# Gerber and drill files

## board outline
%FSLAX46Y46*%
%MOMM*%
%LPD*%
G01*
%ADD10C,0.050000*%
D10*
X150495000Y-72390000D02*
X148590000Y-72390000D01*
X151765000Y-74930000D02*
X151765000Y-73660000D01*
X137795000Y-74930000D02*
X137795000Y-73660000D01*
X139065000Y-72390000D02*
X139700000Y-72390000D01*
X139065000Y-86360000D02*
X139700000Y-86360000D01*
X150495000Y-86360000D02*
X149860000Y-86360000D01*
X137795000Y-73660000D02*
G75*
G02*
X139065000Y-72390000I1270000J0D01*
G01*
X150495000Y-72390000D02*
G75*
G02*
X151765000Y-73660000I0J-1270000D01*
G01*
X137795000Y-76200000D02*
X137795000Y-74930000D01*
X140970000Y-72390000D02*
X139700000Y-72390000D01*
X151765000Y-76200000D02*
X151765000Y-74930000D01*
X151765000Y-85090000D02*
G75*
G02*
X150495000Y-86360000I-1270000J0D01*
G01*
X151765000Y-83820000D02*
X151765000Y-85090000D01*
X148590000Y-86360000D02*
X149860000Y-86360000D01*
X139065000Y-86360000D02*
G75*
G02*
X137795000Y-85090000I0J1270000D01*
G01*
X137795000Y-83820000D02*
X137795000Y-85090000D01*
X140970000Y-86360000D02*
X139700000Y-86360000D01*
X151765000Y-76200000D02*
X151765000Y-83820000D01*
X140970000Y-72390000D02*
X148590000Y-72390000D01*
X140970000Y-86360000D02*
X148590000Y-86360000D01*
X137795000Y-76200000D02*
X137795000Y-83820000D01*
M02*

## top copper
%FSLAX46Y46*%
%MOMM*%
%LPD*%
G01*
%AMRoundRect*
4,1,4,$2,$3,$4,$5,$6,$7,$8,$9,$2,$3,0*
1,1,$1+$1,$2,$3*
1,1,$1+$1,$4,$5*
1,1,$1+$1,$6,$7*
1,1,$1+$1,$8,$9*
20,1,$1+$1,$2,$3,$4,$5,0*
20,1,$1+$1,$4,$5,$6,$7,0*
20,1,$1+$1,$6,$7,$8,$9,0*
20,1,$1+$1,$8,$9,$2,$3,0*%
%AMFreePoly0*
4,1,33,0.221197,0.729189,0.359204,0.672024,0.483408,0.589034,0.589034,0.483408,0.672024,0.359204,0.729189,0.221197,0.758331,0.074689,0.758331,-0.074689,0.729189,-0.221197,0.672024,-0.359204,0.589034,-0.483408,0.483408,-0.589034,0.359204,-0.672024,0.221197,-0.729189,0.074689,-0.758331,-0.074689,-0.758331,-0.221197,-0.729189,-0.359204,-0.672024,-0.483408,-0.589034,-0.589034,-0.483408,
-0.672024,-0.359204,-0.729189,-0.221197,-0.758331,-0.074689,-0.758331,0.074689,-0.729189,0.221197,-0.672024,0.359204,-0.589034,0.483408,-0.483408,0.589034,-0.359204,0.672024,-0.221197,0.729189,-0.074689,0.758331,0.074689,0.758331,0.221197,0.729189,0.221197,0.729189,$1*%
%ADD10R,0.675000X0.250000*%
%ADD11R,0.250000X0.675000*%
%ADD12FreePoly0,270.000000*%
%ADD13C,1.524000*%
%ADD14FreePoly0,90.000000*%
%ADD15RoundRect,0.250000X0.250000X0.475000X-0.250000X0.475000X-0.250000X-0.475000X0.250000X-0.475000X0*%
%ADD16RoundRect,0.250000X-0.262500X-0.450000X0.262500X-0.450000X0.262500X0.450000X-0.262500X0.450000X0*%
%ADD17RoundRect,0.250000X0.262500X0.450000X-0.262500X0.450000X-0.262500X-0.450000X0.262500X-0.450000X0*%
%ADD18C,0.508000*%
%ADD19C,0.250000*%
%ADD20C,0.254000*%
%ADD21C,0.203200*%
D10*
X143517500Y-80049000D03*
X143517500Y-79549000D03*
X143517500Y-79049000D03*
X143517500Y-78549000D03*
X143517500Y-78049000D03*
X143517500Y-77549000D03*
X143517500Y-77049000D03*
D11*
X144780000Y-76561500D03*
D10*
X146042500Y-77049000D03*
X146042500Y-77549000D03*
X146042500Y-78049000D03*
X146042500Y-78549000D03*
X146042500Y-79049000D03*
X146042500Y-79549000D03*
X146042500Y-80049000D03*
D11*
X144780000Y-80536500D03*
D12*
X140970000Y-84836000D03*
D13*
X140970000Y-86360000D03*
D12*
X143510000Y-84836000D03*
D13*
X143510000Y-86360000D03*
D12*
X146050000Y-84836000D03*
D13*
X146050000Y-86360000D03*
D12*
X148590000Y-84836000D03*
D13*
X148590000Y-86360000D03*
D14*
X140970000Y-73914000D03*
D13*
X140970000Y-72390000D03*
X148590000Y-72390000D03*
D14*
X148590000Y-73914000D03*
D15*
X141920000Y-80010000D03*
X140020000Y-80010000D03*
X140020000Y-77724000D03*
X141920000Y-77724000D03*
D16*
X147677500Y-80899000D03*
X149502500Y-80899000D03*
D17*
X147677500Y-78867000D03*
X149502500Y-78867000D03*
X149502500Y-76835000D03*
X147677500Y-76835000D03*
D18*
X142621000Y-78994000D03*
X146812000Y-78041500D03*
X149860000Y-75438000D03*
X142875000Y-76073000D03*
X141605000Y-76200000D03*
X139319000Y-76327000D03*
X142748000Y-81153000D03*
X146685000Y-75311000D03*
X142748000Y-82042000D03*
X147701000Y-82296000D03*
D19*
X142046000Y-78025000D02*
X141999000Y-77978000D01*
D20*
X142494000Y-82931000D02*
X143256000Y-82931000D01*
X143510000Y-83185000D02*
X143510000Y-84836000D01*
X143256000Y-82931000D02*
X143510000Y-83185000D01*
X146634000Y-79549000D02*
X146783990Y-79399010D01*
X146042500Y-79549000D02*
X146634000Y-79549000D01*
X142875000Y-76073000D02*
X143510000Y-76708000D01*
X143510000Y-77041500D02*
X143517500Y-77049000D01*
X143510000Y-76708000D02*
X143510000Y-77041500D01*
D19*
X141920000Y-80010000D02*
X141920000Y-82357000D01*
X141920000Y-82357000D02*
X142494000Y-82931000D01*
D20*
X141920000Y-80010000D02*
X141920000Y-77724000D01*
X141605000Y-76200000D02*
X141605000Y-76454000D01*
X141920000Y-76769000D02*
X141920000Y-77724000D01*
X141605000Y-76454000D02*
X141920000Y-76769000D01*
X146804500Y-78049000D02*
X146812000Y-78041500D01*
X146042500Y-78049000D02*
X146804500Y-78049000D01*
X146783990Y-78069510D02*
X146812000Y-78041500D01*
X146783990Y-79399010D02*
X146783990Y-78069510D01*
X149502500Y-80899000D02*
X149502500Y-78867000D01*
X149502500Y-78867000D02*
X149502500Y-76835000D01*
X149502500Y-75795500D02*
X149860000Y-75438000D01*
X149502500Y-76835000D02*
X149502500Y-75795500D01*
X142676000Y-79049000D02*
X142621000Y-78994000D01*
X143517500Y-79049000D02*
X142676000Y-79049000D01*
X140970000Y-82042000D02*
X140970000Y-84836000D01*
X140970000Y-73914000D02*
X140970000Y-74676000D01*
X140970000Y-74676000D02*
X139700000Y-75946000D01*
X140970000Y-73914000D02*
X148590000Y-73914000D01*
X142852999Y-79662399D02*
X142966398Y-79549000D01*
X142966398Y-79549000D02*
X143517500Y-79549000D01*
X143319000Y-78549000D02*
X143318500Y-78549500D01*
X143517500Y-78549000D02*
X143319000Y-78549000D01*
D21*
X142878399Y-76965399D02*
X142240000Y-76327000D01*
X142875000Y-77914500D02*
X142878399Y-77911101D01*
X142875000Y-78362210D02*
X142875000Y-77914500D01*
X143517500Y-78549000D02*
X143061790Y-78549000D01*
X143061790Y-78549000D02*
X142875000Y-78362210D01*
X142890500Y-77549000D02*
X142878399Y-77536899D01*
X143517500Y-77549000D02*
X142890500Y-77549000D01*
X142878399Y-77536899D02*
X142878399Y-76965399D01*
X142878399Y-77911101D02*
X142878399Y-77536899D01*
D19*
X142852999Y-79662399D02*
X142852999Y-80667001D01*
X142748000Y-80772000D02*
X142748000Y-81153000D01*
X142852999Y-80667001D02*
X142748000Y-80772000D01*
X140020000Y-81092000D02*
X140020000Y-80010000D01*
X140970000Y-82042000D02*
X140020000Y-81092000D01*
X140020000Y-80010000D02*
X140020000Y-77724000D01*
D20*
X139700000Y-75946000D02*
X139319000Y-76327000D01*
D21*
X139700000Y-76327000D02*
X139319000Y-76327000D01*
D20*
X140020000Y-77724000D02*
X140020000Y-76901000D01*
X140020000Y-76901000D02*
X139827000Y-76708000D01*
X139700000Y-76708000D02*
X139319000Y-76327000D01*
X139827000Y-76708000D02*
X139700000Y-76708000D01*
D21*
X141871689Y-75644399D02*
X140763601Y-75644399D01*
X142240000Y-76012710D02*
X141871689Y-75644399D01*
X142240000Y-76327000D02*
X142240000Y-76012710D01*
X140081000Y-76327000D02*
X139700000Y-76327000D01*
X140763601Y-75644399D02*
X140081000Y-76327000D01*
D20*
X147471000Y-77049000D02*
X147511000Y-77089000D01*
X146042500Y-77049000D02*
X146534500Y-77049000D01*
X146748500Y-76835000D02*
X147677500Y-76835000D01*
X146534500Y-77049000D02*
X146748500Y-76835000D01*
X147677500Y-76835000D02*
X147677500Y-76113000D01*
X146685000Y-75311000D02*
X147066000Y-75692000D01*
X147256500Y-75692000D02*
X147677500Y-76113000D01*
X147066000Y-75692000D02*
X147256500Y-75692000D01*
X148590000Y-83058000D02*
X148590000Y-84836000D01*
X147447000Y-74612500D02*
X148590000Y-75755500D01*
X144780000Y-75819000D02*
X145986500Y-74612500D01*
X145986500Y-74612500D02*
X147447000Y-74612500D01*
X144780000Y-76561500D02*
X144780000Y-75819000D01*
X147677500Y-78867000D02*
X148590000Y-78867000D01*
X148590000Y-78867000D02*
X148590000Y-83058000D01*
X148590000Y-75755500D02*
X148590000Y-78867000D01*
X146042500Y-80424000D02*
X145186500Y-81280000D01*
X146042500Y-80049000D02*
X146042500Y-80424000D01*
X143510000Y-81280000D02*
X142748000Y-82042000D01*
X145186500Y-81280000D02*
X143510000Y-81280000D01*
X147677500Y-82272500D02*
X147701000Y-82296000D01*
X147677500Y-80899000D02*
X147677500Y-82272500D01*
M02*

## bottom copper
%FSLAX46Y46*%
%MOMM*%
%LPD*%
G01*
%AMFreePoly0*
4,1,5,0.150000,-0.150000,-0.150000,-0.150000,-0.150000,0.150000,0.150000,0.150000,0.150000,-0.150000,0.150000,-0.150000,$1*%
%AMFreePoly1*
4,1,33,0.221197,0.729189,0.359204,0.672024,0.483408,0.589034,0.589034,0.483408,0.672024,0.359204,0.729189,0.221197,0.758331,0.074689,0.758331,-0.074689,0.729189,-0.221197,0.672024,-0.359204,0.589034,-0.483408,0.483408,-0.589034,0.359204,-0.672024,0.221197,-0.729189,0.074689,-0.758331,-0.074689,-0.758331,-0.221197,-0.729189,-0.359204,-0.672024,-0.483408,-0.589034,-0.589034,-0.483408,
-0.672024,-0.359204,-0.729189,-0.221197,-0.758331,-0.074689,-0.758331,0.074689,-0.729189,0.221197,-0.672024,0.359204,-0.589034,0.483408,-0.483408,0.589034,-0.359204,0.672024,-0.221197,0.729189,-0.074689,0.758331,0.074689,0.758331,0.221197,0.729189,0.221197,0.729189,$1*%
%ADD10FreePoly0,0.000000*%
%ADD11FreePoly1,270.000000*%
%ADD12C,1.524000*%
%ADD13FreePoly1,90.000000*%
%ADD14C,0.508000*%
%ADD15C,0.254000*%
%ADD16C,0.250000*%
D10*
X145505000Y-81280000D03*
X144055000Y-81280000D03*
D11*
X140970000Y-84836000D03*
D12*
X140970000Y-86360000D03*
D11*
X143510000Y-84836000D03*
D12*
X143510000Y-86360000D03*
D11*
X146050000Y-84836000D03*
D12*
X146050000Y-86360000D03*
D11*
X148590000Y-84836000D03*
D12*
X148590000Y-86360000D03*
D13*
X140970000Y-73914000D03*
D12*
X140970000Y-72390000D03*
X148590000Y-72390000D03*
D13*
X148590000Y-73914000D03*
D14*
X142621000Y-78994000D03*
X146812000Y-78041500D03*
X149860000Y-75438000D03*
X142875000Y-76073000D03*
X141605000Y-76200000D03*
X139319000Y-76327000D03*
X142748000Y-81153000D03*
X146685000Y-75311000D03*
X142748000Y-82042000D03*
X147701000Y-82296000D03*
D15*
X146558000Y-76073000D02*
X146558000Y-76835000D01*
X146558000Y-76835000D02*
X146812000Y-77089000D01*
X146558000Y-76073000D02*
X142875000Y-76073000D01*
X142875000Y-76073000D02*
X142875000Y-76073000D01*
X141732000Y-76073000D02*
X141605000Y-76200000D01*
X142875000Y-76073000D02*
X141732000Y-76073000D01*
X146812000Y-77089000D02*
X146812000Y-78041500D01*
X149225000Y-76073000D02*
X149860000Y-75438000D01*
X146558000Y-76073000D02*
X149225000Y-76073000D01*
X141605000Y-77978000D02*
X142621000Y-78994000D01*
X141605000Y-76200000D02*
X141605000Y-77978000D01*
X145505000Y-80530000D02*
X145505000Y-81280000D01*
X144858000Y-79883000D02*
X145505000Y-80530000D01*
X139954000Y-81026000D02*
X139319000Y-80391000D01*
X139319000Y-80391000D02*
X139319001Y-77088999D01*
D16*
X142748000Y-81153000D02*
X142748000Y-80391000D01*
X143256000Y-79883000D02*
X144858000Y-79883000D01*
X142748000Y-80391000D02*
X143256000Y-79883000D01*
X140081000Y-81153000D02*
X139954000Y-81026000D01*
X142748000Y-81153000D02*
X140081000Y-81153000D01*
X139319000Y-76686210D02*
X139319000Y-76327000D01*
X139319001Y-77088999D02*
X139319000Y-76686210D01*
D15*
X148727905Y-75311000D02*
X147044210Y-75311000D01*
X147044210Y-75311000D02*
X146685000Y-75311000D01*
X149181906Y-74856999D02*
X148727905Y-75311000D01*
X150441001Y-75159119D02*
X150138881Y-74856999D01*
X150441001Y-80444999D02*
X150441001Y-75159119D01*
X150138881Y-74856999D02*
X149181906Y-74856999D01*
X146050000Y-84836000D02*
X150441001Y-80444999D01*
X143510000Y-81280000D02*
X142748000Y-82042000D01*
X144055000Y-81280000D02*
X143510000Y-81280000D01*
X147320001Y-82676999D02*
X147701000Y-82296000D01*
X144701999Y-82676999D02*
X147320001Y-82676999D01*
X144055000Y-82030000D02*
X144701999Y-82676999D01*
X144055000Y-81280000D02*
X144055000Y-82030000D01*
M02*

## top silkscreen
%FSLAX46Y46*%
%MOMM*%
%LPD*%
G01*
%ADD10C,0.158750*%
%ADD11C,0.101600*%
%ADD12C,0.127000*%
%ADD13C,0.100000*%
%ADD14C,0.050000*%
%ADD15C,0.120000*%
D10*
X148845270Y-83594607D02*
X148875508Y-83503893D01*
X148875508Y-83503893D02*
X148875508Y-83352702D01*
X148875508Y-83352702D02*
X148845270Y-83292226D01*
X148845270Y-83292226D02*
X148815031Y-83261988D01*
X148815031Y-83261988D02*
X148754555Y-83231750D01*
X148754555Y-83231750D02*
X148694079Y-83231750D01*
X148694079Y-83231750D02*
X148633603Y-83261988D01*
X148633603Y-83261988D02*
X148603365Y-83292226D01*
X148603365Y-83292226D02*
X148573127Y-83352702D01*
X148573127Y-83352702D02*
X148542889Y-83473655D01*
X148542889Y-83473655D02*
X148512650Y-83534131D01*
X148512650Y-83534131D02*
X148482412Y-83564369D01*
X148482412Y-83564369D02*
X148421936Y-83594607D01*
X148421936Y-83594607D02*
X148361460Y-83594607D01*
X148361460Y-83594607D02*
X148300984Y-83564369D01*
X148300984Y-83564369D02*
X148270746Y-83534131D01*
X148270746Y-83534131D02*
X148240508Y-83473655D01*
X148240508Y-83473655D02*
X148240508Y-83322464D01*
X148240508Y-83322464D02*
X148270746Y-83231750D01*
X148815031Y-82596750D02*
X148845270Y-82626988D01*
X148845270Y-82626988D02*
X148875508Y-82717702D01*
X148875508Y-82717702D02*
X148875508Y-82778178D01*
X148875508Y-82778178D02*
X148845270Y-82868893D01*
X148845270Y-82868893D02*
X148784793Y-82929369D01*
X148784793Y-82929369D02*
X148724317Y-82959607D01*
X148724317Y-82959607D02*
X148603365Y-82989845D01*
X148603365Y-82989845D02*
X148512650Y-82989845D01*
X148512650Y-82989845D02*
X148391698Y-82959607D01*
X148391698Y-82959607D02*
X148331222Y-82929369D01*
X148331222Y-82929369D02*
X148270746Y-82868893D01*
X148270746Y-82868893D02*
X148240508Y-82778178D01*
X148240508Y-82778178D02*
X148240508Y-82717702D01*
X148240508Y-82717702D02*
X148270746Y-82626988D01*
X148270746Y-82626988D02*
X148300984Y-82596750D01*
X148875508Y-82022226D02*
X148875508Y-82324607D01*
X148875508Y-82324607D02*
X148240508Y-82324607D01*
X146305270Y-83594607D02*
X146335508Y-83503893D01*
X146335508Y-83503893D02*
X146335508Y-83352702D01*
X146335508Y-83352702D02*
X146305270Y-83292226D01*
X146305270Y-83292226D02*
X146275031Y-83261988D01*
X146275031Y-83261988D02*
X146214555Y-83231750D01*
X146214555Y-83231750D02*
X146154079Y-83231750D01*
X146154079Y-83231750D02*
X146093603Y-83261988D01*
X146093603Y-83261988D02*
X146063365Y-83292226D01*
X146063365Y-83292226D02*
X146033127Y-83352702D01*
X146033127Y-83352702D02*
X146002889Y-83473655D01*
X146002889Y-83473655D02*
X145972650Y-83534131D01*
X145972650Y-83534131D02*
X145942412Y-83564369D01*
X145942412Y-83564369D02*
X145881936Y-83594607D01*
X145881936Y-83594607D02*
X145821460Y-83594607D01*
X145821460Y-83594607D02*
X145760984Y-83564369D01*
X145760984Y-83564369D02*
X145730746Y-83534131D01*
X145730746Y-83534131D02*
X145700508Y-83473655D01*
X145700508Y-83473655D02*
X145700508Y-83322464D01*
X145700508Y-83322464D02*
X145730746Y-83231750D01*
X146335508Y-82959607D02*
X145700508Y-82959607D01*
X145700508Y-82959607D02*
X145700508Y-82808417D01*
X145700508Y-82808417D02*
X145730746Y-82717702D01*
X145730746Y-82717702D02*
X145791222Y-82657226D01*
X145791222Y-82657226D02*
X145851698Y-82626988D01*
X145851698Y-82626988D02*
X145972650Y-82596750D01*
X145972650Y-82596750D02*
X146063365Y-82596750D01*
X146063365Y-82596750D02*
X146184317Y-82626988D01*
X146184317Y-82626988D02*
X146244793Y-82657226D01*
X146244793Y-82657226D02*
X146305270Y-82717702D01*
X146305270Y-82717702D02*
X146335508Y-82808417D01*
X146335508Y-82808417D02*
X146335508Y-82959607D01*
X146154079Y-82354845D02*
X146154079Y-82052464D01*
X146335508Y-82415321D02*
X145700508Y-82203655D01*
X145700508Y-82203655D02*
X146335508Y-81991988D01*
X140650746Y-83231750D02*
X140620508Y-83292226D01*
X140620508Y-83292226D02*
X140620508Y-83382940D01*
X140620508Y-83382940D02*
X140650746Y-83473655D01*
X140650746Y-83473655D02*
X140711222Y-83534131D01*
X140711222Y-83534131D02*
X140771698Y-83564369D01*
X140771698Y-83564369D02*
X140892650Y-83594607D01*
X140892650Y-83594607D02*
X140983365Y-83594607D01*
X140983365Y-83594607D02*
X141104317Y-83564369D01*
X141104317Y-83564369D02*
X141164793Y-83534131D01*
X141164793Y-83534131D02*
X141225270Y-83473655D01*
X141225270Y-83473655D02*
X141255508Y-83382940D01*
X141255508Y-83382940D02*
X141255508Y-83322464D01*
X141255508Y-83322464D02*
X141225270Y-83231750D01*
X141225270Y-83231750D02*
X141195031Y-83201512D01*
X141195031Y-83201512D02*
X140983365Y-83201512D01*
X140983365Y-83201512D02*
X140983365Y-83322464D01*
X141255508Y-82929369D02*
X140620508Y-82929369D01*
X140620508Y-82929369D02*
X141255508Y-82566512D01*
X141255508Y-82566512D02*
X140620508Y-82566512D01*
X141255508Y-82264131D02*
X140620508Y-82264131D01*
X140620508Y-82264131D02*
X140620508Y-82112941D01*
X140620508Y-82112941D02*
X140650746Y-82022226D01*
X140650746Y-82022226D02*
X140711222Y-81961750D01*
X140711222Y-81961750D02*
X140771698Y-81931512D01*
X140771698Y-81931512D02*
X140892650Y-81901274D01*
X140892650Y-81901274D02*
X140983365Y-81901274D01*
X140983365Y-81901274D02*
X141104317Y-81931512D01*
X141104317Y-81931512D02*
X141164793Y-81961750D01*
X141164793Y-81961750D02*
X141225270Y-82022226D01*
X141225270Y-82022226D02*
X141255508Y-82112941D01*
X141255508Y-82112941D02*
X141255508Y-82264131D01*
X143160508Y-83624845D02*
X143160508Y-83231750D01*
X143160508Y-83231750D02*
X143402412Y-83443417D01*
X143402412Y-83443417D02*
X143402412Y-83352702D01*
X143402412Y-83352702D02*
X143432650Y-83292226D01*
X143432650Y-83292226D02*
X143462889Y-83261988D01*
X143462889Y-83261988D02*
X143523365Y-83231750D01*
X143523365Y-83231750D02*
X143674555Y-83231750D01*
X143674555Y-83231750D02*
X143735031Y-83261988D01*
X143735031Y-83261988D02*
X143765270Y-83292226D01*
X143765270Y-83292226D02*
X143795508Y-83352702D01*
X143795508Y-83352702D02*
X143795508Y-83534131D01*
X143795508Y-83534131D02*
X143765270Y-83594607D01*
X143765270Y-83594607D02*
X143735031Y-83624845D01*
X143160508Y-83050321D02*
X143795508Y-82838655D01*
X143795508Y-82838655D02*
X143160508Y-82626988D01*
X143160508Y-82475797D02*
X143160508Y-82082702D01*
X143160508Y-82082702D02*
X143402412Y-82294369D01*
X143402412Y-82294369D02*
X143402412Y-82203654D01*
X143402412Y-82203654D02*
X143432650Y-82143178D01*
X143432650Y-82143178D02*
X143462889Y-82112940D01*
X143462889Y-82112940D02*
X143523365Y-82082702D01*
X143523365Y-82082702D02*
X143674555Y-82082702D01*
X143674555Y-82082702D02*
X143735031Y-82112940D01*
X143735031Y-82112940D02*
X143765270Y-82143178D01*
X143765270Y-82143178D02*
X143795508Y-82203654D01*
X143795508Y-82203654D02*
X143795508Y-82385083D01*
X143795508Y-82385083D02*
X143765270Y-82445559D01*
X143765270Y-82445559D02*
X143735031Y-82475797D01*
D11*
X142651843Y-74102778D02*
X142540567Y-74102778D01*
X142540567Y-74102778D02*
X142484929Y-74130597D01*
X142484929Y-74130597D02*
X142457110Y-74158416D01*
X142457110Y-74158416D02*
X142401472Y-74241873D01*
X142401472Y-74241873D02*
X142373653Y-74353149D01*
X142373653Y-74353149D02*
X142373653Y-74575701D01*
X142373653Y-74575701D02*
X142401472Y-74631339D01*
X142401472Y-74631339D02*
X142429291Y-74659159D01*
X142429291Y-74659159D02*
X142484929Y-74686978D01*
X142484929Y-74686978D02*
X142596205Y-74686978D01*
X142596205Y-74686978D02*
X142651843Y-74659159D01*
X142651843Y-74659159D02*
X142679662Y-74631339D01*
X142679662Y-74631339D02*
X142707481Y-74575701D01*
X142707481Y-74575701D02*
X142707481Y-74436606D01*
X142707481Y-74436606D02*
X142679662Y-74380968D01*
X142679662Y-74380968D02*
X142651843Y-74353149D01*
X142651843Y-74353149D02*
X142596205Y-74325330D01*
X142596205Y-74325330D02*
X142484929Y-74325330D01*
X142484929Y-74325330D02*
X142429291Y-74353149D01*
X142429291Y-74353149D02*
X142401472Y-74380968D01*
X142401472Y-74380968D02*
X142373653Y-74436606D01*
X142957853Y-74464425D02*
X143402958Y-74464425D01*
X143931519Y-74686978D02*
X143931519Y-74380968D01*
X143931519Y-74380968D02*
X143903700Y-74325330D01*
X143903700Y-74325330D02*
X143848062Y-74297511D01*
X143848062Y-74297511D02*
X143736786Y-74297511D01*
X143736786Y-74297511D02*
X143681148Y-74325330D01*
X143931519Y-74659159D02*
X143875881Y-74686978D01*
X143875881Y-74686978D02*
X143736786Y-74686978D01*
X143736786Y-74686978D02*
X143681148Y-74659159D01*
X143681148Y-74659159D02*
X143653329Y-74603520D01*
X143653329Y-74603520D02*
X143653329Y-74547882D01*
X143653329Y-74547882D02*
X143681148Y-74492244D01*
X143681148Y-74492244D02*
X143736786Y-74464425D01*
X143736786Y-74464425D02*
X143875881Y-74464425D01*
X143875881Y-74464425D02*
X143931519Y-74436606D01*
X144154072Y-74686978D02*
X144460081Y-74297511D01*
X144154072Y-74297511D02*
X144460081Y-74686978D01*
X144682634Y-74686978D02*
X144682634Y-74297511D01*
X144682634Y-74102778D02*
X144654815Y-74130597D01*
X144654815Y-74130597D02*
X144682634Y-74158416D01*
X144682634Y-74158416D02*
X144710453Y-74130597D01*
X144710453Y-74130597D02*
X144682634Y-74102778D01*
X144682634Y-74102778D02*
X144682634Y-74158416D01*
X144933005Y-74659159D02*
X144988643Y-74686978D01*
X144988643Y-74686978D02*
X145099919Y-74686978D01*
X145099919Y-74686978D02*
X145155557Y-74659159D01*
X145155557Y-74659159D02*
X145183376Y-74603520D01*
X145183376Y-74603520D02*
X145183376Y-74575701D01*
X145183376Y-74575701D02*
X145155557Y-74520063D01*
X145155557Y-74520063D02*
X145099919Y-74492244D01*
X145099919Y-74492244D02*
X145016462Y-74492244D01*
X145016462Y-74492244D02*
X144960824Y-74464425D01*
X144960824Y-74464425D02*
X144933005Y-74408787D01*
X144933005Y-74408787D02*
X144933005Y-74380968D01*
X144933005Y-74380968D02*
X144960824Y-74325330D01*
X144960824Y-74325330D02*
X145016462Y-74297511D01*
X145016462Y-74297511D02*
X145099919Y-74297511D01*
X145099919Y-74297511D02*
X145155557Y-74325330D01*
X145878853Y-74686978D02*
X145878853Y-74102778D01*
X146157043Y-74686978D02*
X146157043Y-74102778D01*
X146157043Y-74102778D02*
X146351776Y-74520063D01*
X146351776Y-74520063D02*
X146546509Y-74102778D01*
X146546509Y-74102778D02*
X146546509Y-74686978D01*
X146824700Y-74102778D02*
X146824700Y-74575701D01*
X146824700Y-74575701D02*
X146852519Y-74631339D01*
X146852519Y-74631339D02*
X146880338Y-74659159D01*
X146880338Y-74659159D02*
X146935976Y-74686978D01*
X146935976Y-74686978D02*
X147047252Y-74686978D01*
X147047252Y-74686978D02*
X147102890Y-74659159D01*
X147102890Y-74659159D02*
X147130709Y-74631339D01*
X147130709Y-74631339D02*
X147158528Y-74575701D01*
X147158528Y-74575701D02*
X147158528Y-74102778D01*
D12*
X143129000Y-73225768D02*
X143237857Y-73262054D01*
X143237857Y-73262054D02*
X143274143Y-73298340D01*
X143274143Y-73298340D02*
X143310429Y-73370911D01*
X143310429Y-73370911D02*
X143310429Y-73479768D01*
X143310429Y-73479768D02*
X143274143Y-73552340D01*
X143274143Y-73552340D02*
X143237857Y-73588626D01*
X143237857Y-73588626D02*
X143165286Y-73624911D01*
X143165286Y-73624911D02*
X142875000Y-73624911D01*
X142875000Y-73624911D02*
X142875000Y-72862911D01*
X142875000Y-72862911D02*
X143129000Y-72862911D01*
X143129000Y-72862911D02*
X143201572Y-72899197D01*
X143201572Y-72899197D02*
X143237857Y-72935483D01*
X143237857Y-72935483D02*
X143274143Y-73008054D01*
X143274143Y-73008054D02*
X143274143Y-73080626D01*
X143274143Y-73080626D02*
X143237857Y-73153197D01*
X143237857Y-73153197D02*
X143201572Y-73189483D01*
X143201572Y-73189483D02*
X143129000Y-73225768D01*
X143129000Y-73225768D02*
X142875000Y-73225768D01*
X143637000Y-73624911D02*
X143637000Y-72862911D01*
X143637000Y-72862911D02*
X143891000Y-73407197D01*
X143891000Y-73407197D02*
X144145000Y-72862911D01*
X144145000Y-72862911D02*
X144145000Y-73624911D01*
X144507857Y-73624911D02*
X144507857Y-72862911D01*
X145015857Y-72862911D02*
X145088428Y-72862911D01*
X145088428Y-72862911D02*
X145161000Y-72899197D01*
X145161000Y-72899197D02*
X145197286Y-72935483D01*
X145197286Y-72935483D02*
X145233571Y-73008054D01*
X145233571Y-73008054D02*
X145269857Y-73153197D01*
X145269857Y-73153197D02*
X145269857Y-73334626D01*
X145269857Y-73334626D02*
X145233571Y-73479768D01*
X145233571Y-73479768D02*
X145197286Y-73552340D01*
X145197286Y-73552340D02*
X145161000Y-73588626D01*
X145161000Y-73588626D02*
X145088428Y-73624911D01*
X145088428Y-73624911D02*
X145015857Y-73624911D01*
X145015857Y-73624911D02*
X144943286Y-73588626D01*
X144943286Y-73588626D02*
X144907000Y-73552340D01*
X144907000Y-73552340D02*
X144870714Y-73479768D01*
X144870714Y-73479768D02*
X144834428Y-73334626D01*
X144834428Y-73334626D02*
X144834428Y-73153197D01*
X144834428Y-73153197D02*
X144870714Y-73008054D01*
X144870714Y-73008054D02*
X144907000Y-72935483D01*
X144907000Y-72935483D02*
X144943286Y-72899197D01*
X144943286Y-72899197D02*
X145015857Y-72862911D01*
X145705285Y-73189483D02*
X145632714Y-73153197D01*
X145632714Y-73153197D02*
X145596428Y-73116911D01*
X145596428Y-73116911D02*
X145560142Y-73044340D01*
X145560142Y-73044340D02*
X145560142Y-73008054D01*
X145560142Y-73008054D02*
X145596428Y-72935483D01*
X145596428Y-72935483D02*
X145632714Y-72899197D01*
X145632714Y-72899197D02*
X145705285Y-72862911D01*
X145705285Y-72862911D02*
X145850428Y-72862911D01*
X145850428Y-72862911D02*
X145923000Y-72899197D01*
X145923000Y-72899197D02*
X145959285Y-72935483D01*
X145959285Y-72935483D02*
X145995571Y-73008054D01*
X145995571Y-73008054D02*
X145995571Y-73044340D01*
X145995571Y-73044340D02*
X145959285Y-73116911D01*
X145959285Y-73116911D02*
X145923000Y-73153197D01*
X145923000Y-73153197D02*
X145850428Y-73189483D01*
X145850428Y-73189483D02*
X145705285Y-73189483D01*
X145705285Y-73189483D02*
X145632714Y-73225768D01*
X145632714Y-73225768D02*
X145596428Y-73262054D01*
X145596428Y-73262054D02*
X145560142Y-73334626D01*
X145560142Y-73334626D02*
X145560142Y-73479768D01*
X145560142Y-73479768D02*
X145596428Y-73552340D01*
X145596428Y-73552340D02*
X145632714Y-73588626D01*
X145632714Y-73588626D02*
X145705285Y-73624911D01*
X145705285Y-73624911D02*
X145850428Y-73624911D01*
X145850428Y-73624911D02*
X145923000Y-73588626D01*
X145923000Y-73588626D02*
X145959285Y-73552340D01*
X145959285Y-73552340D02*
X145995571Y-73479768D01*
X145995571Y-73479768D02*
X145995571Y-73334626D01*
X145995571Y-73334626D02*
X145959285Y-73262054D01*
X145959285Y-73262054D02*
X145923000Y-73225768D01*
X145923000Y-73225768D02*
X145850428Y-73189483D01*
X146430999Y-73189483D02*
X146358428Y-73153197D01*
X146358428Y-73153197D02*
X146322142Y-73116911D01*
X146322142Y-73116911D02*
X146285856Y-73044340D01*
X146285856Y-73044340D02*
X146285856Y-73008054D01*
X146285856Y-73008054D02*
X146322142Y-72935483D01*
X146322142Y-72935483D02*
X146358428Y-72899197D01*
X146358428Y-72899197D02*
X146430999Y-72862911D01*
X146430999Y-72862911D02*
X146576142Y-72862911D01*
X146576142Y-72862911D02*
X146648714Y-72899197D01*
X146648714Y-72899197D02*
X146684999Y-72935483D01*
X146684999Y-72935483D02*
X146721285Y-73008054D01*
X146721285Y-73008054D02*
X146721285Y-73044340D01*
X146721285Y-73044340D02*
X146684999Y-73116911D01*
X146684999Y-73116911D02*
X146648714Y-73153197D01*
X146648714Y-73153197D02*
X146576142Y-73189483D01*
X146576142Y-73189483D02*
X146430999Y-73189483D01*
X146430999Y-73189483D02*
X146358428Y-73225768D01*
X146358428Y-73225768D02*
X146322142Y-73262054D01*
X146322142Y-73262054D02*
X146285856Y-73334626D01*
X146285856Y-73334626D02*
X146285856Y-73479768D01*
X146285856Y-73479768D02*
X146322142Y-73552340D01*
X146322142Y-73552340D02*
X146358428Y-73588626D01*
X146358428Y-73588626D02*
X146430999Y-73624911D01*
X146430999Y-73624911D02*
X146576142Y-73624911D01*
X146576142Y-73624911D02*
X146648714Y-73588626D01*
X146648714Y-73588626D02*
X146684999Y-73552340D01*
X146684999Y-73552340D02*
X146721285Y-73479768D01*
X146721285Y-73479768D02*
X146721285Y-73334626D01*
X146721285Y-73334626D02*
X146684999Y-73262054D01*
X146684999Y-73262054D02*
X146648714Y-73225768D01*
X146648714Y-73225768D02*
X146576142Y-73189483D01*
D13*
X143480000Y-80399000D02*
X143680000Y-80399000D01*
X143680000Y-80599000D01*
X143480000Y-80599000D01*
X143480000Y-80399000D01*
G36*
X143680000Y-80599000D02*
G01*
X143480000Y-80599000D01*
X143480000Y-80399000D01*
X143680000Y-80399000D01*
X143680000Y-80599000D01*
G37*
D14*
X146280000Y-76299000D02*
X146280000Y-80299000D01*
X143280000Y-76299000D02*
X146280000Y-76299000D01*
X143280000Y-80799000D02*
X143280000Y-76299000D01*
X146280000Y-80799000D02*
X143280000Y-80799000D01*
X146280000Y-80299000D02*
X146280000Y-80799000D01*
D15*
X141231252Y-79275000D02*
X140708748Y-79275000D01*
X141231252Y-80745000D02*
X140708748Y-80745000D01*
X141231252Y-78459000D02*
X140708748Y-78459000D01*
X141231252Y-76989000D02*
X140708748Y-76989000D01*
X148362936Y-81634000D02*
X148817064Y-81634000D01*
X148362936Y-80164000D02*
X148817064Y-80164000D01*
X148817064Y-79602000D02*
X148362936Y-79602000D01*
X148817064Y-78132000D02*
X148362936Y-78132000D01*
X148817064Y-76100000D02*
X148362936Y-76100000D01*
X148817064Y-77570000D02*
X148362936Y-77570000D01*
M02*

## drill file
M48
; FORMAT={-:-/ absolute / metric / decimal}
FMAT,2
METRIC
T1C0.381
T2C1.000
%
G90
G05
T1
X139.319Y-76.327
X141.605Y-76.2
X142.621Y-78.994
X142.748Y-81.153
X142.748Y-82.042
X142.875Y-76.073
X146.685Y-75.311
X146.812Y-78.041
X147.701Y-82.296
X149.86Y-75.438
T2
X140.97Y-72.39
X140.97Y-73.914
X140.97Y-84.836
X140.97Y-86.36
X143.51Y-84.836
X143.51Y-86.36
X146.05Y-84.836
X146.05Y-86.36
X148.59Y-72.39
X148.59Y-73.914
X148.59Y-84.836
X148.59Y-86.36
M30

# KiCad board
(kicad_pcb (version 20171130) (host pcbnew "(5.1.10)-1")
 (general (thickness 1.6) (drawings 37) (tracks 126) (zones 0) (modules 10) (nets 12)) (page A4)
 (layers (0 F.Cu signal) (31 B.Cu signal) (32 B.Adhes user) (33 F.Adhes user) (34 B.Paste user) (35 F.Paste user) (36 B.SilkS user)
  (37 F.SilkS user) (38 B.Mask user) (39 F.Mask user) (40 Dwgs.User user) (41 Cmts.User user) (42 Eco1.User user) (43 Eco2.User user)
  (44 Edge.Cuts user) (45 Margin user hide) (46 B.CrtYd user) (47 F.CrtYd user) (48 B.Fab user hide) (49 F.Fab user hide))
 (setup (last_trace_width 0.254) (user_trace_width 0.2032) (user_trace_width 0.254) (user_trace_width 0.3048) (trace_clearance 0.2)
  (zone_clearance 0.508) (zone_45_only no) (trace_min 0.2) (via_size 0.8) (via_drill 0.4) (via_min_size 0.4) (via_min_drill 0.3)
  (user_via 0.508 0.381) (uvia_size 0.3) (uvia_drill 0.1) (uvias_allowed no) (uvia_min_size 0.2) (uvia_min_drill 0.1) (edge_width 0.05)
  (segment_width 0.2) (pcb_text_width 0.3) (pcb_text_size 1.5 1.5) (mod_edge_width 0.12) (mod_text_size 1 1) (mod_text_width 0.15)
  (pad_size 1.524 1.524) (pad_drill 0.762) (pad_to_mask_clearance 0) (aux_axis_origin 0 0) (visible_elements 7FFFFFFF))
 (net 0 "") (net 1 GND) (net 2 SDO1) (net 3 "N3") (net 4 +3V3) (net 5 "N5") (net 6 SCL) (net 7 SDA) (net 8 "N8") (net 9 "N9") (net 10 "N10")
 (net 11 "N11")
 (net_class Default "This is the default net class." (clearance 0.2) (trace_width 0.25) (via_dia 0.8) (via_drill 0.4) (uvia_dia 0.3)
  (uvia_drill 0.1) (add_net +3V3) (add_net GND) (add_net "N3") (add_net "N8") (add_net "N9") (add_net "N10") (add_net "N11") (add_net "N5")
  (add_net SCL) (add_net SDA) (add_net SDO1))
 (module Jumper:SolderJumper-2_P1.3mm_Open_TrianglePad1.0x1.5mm (layer B.Cu) (at 144.78 81.28)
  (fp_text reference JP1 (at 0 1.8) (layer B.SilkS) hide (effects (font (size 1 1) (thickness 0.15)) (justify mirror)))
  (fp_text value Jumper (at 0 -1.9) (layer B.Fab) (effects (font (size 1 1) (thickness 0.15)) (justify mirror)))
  (pad 2 smd custom (at 0.725 0) (size 0.3 0.3) (layers B.Cu B.Mask) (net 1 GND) (zone_connect 2)
   (options (clearance outline) (anchor rect)) (primitives))
  (pad 1 smd custom (at -0.725 0) (size 0.3 0.3) (layers B.Cu B.Mask) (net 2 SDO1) (zone_connect 2)
   (options (clearance outline) (anchor rect)) (primitives)))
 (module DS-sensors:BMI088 (layer F.Cu) (at 144.78 80.899 180)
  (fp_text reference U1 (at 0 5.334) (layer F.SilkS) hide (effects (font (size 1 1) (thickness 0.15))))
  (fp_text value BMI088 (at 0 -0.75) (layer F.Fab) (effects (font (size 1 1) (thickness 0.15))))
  (fp_poly (pts (xy 1.3 0.5) (xy 1.1 0.5) (xy 1.1 0.3) (xy 1.3 0.3)) (layer F.SilkS) (width 0.1))
  (fp_line (start -1.5 4.6) (end -1.5 0.6) (layer F.SilkS) (width 0.05))
  (fp_line (start 1.5 4.6) (end -1.5 4.6) (layer F.SilkS) (width 0.05))
  (fp_line (start 1.5 0.1) (end 1.5 4.6) (layer F.SilkS) (width 0.05))
  (fp_line (start -1.5 0.1) (end 1.5 0.1) (layer F.SilkS) (width 0.05))
  (fp_line (start -1.5 0.6) (end -1.5 0.1) (layer F.SilkS) (width 0.05))
  (pad 1 smd rect (at 1.2625 0.85 180) (size 0.675 0.25) (layers F.Cu F.Paste F.Mask) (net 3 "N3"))
  (pad 2 smd rect (at 1.2625 1.35 180) (size 0.675 0.25) (layers F.Cu F.Paste F.Mask) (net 1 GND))
  (pad 3 smd rect (at 1.2625 1.85 180) (size 0.675 0.25) (layers F.Cu F.Paste F.Mask) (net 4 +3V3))
  (pad 4 smd rect (at 1.2625 2.35 180) (size 0.675 0.25) (layers F.Cu F.Paste F.Mask) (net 1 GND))
  (pad 5 smd rect (at 1.2625 2.85 180) (size 0.675 0.25) (layers F.Cu F.Paste F.Mask) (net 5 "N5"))
  (pad 6 smd rect (at 1.2625 3.35 180) (size 0.675 0.25) (layers F.Cu F.Paste F.Mask) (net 1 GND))
  (pad 7 smd rect (at 1.2625 3.85 180) (size 0.675 0.25) (layers F.Cu F.Paste F.Mask) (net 4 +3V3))
  (pad 8 smd rect (at 0 4.3375 270) (size 0.675 0.25) (layers F.Cu F.Paste F.Mask) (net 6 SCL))
  (pad 9 smd rect (at -1.2625 3.85) (size 0.675 0.25) (layers F.Cu F.Paste F.Mask) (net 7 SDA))
  (pad 10 smd rect (at -1.2625 3.35) (size 0.675 0.25) (layers F.Cu F.Paste F.Mask) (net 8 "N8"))
  (pad 11 smd rect (at -1.2625 2.85) (size 0.675 0.25) (layers F.Cu F.Paste F.Mask) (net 4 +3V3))
  (pad 12 smd rect (at -1.2625 2.35) (size 0.675 0.25) (layers F.Cu F.Paste F.Mask) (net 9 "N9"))
  (pad 13 smd rect (at -1.2625 1.85) (size 0.675 0.25) (layers F.Cu F.Paste F.Mask) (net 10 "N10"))
  (pad 14 smd rect (at -1.2625 1.35) (size 0.675 0.25) (layers F.Cu F.Paste F.Mask) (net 4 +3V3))
  (pad 15 smd rect (at -1.2625 0.85) (size 0.675 0.25) (layers F.Cu F.Paste F.Mask) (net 2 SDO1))
  (pad 16 smd rect (at 0 0.3625 90) (size 0.675 0.25) (layers F.Cu F.Paste F.Mask) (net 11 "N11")))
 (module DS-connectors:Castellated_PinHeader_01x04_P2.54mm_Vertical (layer B.Cu) (at 138.43 84.836 270)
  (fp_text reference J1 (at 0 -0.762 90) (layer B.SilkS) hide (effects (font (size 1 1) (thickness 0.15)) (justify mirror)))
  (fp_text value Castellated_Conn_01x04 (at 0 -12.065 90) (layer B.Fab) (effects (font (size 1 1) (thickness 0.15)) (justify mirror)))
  (pad 1 thru_hole custom (at 0 -2.54 270) (size 1.524 1.524) (drill 1) (layers *.Cu *.Mask) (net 1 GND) (zone_connect 0)
   (options (clearance outline) (anchor circle)) (primitives))
  (pad 1 thru_hole circle (at 1.524 -2.54 270) (size 1.524 1.524) (drill 1) (layers *.Cu *.Mask) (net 1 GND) (zone_connect 0))
  (pad 2 thru_hole custom (at 0 -5.08 270) (size 1.524 1.524) (drill 1) (layers *.Cu *.Mask) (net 4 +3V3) (zone_connect 0)
   (options (clearance outline) (anchor circle)) (primitives))
  (pad 2 thru_hole circle (at 1.524 -5.08 270) (size 1.524 1.524) (drill 1) (layers *.Cu *.Mask) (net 4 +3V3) (zone_connect 0))
  (pad 3 thru_hole custom (at 0 -7.62 270) (size 1.524 1.524) (drill 1) (layers *.Cu *.Mask) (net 7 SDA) (zone_connect 0)
   (options (clearance outline) (anchor circle)) (primitives))
  (pad 3 thru_hole circle (at 1.524 -7.62 270) (size 1.524 1.524) (drill 1) (layers *.Cu *.Mask) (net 7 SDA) (zone_connect 0))
  (pad 4 thru_hole custom (at 0 -10.16 270) (size 1.524 1.524) (drill 1) (layers *.Cu *.Mask) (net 6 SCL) (zone_connect 0)
   (options (clearance outline) (anchor circle)) (primitives))
  (pad 4 thru_hole circle (at 1.524 -10.16 270) (size 1.524 1.524) (drill 1) (layers *.Cu *.Mask) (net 6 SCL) (zone_connect 0)))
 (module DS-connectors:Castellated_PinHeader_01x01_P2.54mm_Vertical (layer F.Cu) (at 138.938 73.914 90)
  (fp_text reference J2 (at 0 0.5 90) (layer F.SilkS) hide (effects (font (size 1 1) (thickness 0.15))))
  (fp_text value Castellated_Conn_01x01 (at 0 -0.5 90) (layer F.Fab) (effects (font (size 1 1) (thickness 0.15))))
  (pad 1 thru_hole custom (at 0 2.032 90) (size 1.524 1.524) (drill 1) (layers *.Cu *.Mask) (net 1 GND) (zone_connect 0)
   (options (clearance outline) (anchor circle)) (primitives))
  (pad 1 thru_hole circle (at 1.524 2.032 90) (size 1.524 1.524) (drill 1) (layers *.Cu *.Mask) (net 1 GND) (zone_connect 0)))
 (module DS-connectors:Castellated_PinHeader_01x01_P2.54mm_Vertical (layer F.Cu) (at 146.558 73.914 90)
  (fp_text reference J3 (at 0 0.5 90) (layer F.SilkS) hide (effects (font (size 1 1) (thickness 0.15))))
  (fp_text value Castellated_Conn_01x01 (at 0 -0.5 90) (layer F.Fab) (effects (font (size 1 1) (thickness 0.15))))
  (pad 1 thru_hole circle (at 1.524 2.032 90) (size 1.524 1.524) (drill 1) (layers *.Cu *.Mask) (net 1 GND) (zone_connect 0))
  (pad 1 thru_hole custom (at 0 2.032 90) (size 1.524 1.524) (drill 1) (layers *.Cu *.Mask) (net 1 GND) (zone_connect 0)
   (options (clearance outline) (anchor circle)) (primitives)))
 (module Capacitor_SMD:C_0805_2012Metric (layer F.Cu) (at 140.97 80.01 180)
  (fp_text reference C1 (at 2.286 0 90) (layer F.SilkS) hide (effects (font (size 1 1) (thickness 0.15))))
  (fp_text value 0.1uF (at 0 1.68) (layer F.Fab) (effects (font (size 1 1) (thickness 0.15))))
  (fp_line (start -0.261252 0.735) (end 0.261252 0.735) (layer F.SilkS) (width 0.12))
  (fp_line (start -0.261252 -0.735) (end 0.261252 -0.735) (layer F.SilkS) (width 0.12))
  (pad 1 smd roundrect (at -0.95 0 180) (size 1 1.45) (layers F.Cu F.Paste F.Mask) (roundrect_rratio 0.25) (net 4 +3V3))
  (pad 2 smd roundrect (at 0.95 0 180) (size 1 1.45) (layers F.Cu F.Paste F.Mask) (roundrect_rratio 0.25) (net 1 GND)))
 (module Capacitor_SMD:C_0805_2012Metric (layer F.Cu) (at 140.97 77.724 180)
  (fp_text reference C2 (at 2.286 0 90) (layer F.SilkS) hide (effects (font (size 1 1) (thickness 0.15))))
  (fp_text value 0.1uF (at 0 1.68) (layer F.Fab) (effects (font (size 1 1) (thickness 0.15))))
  (fp_line (start -0.261252 -0.735) (end 0.261252 -0.735) (layer F.SilkS) (width 0.12))
  (fp_line (start -0.261252 0.735) (end 0.261252 0.735) (layer F.SilkS) (width 0.12))
  (pad 2 smd roundrect (at 0.95 0 180) (size 1 1.45) (layers F.Cu F.Paste F.Mask) (roundrect_rratio 0.25) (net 1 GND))
  (pad 1 smd roundrect (at -0.95 0 180) (size 1 1.45) (layers F.Cu F.Paste F.Mask) (roundrect_rratio 0.25) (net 4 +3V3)))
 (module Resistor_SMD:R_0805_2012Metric (layer F.Cu) (at 148.59 80.899)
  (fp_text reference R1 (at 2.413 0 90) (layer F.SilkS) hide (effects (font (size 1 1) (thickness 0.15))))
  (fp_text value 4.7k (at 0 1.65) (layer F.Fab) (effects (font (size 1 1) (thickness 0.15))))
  (fp_line (start -0.227064 0.735) (end 0.227064 0.735) (layer F.SilkS) (width 0.12))
  (fp_line (start -0.227064 -0.735) (end 0.227064 -0.735) (layer F.SilkS) (width 0.12))
  (pad 1 smd roundrect (at -0.9125 0) (size 1.025 1.4) (layers F.Cu F.Paste F.Mask) (roundrect_rratio 0.243902) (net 2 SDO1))
  (pad 2 smd roundrect (at 0.9125 0) (size 1.025 1.4) (layers F.Cu F.Paste F.Mask) (roundrect_rratio 0.243902) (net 4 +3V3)))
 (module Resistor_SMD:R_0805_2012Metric (layer F.Cu) (at 148.59 78.867 180)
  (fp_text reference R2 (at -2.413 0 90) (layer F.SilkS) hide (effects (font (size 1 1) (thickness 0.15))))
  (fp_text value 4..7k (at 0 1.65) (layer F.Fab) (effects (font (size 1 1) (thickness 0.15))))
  (fp_line (start -0.227064 -0.735) (end 0.227064 -0.735) (layer F.SilkS) (width 0.12))
  (fp_line (start -0.227064 0.735) (end 0.227064 0.735) (layer F.SilkS) (width 0.12))
  (pad 2 smd roundrect (at 0.9125 0 180) (size 1.025 1.4) (layers F.Cu F.Paste F.Mask) (roundrect_rratio 0.243902) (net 6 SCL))
  (pad 1 smd roundrect (at -0.9125 0 180) (size 1.025 1.4) (layers F.Cu F.Paste F.Mask) (roundrect_rratio 0.243902) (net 4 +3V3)))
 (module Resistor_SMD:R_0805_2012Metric (layer F.Cu) (at 148.59 76.835 180)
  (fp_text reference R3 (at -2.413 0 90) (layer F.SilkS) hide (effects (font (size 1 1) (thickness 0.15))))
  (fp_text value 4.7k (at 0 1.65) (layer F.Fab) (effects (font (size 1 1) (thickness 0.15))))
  (fp_line (start -0.227064 0.735) (end 0.227064 0.735) (layer F.SilkS) (width 0.12))
  (fp_line (start -0.227064 -0.735) (end 0.227064 -0.735) (layer F.SilkS) (width 0.12))
  (pad 1 smd roundrect (at -0.9125 0 180) (size 1.025 1.4) (layers F.Cu F.Paste F.Mask) (roundrect_rratio 0.243902) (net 4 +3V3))
  (pad 2 smd roundrect (at 0.9125 0 180) (size 1.025 1.4) (layers F.Cu F.Paste F.Mask) (roundrect_rratio 0.243902) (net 7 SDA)))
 (gr_line (start 150.495 72.39) (end 148.59 72.39) (layer Edge.Cuts) (width 0.05))
 (gr_line (start 151.765 74.93) (end 151.765 73.66) (layer Edge.Cuts) (width 0.05))
 (gr_line (start 137.795 74.93) (end 137.795 73.66) (layer Edge.Cuts) (width 0.05))
 (gr_line (start 139.065 72.39) (end 139.7 72.39) (layer Edge.Cuts) (width 0.05))
 (gr_line (start 139.065 86.36) (end 139.7 86.36) (layer Edge.Cuts) (width 0.05))
 (gr_line (start 150.495 86.36) (end 149.86 86.36) (layer Edge.Cuts) (width 0.05))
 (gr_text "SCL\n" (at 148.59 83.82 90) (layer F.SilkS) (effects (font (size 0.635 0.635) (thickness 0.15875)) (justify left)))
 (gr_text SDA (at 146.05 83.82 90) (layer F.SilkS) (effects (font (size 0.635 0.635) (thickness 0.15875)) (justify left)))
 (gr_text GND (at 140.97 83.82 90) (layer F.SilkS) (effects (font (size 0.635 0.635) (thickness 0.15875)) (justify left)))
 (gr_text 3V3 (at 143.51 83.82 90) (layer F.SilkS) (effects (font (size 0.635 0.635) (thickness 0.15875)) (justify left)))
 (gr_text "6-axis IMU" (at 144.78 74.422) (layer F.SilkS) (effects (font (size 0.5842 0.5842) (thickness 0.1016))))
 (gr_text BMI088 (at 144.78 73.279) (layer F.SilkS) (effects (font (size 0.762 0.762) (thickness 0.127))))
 (gr_arc (start 139.065 73.66) (end 139.065 72.39) (angle -90) (layer Edge.Cuts) (width 0.05))
 (gr_arc (start 150.495 73.66) (end 151.765 73.66) (angle -90) (layer Edge.Cuts) (width 0.05))
 (gr_line (start 137.795 76.2) (end 137.795 74.93) (layer Edge.Cuts) (width 0.05))
 (gr_line (start 140.97 72.39) (end 139.7 72.39) (layer Edge.Cuts) (width 0.05))
 (gr_line (start 151.765 76.2) (end 151.765 74.93) (layer Edge.Cuts) (width 0.05))
 (gr_arc (start 150.495 85.09) (end 150.495 86.36) (angle -90) (layer Edge.Cuts) (width 0.05))
 (gr_line (start 151.765 83.82) (end 151.765 85.09) (layer Edge.Cuts) (width 0.05))
 (gr_line (start 148.59 86.36) (end 149.86 86.36) (layer Edge.Cuts) (width 0.05))
 (gr_arc (start 139.065 85.09) (end 137.795 85.09) (angle -90) (layer Edge.Cuts) (width 0.05))
 (gr_line (start 137.795 83.82) (end 137.795 85.09) (layer Edge.Cuts) (width 0.05))
 (gr_line (start 140.97 86.36) (end 139.7 86.36) (layer Edge.Cuts) (width 0.05))
 (gr_line (start 151.765 76.2) (end 151.765 83.82) (layer Edge.Cuts) (width 0.05))
 (gr_line (start 140.97 72.39) (end 148.59 72.39) (layer Edge.Cuts) (width 0.05))
 (gr_line (start 140.97 86.36) (end 148.59 86.36) (layer Edge.Cuts) (width 0.05))
 (gr_line (start 137.795 76.2) (end 137.795 83.82) (layer Edge.Cuts) (width 0.05))
 (via (at 142.621 78.994) (size 0.508) (drill 0.381) (layers F.Cu B.Cu) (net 4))
 (via (at 146.812 78.0415) (size 0.508) (drill 0.381) (layers F.Cu B.Cu) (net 4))
 (via (at 149.86 75.438) (size 0.508) (drill 0.381) (layers F.Cu B.Cu) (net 4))
 (segment (start 142.046 78.025) (end 141.999 77.978) (width 0.25) (layer F.Cu) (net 4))
 (segment (start 142.494 82.931) (end 143.256 82.931) (width 0.254) (layer F.Cu) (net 4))
 (segment (start 143.51 83.185) (end 143.51 84.836) (width 0.254) (layer F.Cu) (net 4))
 (segment (start 143.256 82.931) (end 143.51 83.185) (width 0.254) (layer F.Cu) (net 4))
 (segment (start 146.558 76.073) (end 146.558 76.835) (width 0.254) (layer B.Cu) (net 4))
 (segment (start 146.558 76.835) (end 146.812 77.089) (width 0.254) (layer B.Cu) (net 4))
 (segment (start 146.634 79.549) (end 146.78399 79.39901) (width 0.254) (layer F.Cu) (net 4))
 (segment (start 146.0425 79.549) (end 146.634 79.549) (width 0.254) (layer F.Cu) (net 4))
 (segment (start 146.558 76.073) (end 142.875 76.073) (width 0.254) (layer B.Cu) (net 4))
 (segment (start 142.875 76.073) (end 142.875 76.073) (width 0.254) (layer B.Cu) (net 4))
 (via (at 142.875 76.073) (size 0.508) (drill 0.381) (layers F.Cu B.Cu) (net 4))
 (segment (start 142.875 76.073) (end 143.51 76.708) (width 0.254) (layer F.Cu) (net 4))
 (segment (start 143.51 77.0415) (end 143.5175 77.049) (width 0.254) (layer F.Cu) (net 4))
 (segment (start 143.51 76.708) (end 143.51 77.0415) (width 0.254) (layer F.Cu) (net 4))
 (via (at 141.605 76.2) (size 0.508) (drill 0.381) (layers F.Cu B.Cu) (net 4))
 (segment (start 141.92 80.01) (end 141.92 82.357) (width 0.25) (layer F.Cu) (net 4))
 (segment (start 141.92 82.357) (end 142.494 82.931) (width 0.25) (layer F.Cu) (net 4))
 (segment (start 141.92 80.01) (end 141.92 77.724) (width 0.254) (layer F.Cu) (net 4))
 (segment (start 141.605 76.2) (end 141.605 76.454) (width 0.254) (layer F.Cu) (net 4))
 (segment (start 141.92 76.769) (end 141.92 77.724) (width 0.254) (layer F.Cu) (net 4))
 (segment (start 141.605 76.454) (end 141.92 76.769) (width 0.254) (layer F.Cu) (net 4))
 (segment (start 141.732 76.073) (end 141.605 76.2) (width 0.254) (layer B.Cu) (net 4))
 (segment (start 142.875 76.073) (end 141.732 76.073) (width 0.254) (layer B.Cu) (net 4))
 (segment (start 146.8045 78.049) (end 146.812 78.0415) (width 0.254) (layer F.Cu) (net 4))
 (segment (start 146.0425 78.049) (end 146.8045 78.049) (width 0.254) (layer F.Cu) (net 4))
 (segment (start 146.812 77.089) (end 146.812 78.0415) (width 0.254) (layer B.Cu) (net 4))
 (segment (start 146.78399 78.06951) (end 146.812 78.0415) (width 0.254) (layer F.Cu) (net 4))
 (segment (start 146.78399 79.39901) (end 146.78399 78.06951) (width 0.254) (layer F.Cu) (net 4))
 (segment (start 149.5025 80.899) (end 149.5025 78.867) (width 0.254) (layer F.Cu) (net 4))
 (segment (start 149.5025 78.867) (end 149.5025 76.835) (width 0.254) (layer F.Cu) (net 4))
 (segment (start 149.225 76.073) (end 149.86 75.438) (width 0.254) (layer B.Cu) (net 4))
 (segment (start 146.558 76.073) (end 149.225 76.073) (width 0.254) (layer B.Cu) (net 4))
 (segment (start 149.5025 75.7955) (end 149.86 75.438) (width 0.254) (layer F.Cu) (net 4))
 (segment (start 149.5025 76.835) (end 149.5025 75.7955) (width 0.254) (layer F.Cu) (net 4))
 (segment (start 142.676 79.049) (end 142.621 78.994) (width 0.254) (layer F.Cu) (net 4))
 (segment (start 143.5175 79.049) (end 142.676 79.049) (width 0.254) (layer F.Cu) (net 4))
 (segment (start 141.605 77.978) (end 142.621 78.994) (width 0.254) (layer B.Cu) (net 4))
 (segment (start 141.605 76.2) (end 141.605 77.978) (width 0.254) (layer B.Cu) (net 4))
 (via (at 139.319 76.327) (size 0.508) (drill 0.381) (layers F.Cu B.Cu) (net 1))
 (via (at 142.748 81.153) (size 0.508) (drill 0.381) (layers F.Cu B.Cu) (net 1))
 (segment (start 145.505 80.53) (end 145.505 81.28) (width 0.254) (layer B.Cu) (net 1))
 (segment (start 144.858 79.883) (end 145.505 80.53) (width 0.254) (layer B.Cu) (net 1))
 (segment (start 139.954 81.026) (end 139.319 80.391) (width 0.254) (layer B.Cu) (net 1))
 (segment (start 139.319 80.391) (end 139.319001 77.088999) (width 0.254) (layer B.Cu) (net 1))
 (segment (start 140.97 82.042) (end 140.97 84.836) (width 0.254) (layer F.Cu) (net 1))
 (segment (start 140.97 73.914) (end 140.97 74.676) (width 0.254) (layer F.Cu) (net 1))
 (segment (start 140.97 74.676) (end 139.7 75.946) (width 0.254) (layer F.Cu) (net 1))
 (segment (start 140.97 73.914) (end 148.59 73.914) (width 0.254) (layer F.Cu) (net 1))
 (segment (start 142.852999 79.662399) (end 142.966398 79.549) (width 0.254) (layer F.Cu) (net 1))
 (segment (start 142.966398 79.549) (end 143.5175 79.549) (width 0.254) (layer F.Cu) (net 1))
 (segment (start 143.319 78.549) (end 143.3185 78.5495) (width 0.254) (layer F.Cu) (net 1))
 (segment (start 143.5175 78.549) (end 143.319 78.549) (width 0.254) (layer F.Cu) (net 1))
 (segment (start 142.878399 76.965399) (end 142.24 76.327) (width 0.2032) (layer F.Cu) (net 1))
 (segment (start 142.875 77.9145) (end 142.878399 77.911101) (width 0.2032) (layer F.Cu) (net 1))
 (segment (start 142.875 78.36221) (end 142.875 77.9145) (width 0.2032) (layer F.Cu) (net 1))
 (segment (start 143.5175 78.549) (end 143.06179 78.549) (width 0.2032) (layer F.Cu) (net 1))
 (segment (start 143.06179 78.549) (end 142.875 78.36221) (width 0.2032) (layer F.Cu) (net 1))
 (segment (start 142.8905 77.549) (end 142.878399 77.536899) (width 0.2032) (layer F.Cu) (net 1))
 (segment (start 143.5175 77.549) (end 142.8905 77.549) (width 0.2032) (layer F.Cu) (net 1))
 (segment (start 142.878399 77.536899) (end 142.878399 76.965399) (width 0.2032) (layer F.Cu) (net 1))
 (segment (start 142.878399 77.911101) (end 142.878399 77.536899) (width 0.2032) (layer F.Cu) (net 1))
 (segment (start 142.748 81.153) (end 142.748 80.391) (width 0.25) (layer B.Cu) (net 1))
 (segment (start 143.256 79.883) (end 144.858 79.883) (width 0.25) (layer B.Cu) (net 1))
 (segment (start 142.748 80.391) (end 143.256 79.883) (width 0.25) (layer B.Cu) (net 1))
 (segment (start 142.852999 79.662399) (end 142.852999 80.667001) (width 0.25) (layer F.Cu) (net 1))
 (segment (start 142.748 80.772) (end 142.748 81.153) (width 0.25) (layer F.Cu) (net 1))
 (segment (start 142.852999 80.667001) (end 142.748 80.772) (width 0.25) (layer F.Cu) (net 1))
 (segment (start 140.081 81.153) (end 139.954 81.026) (width 0.25) (layer B.Cu) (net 1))
 (segment (start 142.748 81.153) (end 140.081 81.153) (width 0.25) (layer B.Cu) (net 1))
 (segment (start 140.02 81.092) (end 140.02 80.01) (width 0.25) (layer F.Cu) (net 1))
 (segment (start 140.97 82.042) (end 140.02 81.092) (width 0.25) (layer F.Cu) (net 1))
 (segment (start 140.02 80.01) (end 140.02 77.724) (width 0.25) (layer F.Cu) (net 1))
 (segment (start 139.319 76.68621) (end 139.319 76.327) (width 0.25) (layer B.Cu) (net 1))
 (segment (start 139.319001 77.088999) (end 139.319 76.68621) (width 0.25) (layer B.Cu) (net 1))
 (segment (start 139.7 75.946) (end 139.319 76.327) (width 0.254) (layer F.Cu) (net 1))
 (segment (start 139.7 76.327) (end 139.319 76.327) (width 0.2032) (layer F.Cu) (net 1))
 (segment (start 140.02 77.724) (end 140.02 76.901) (width 0.254) (layer F.Cu) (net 1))
 (segment (start 140.02 76.901) (end 139.827 76.708) (width 0.254) (layer F.Cu) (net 1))
 (segment (start 139.7 76.708) (end 139.319 76.327) (width 0.254) (layer F.Cu) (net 1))
 (segment (start 139.827 76.708) (end 139.7 76.708) (width 0.254) (layer F.Cu) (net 1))
 (segment (start 141.871689 75.644399) (end 140.763601 75.644399) (width 0.2032) (layer F.Cu) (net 1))
 (segment (start 142.24 76.01271) (end 141.871689 75.644399) (width 0.2032) (layer F.Cu) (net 1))
 (segment (start 142.24 76.327) (end 142.24 76.01271) (width 0.2032) (layer F.Cu) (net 1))
 (segment (start 140.081 76.327) (end 139.7 76.327) (width 0.2032) (layer F.Cu) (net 1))
 (segment (start 140.763601 75.644399) (end 140.081 76.327) (width 0.2032) (layer F.Cu) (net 1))
 (via (at 146.685 75.311) (size 0.508) (drill 0.381) (layers F.Cu B.Cu) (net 7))
 (segment (start 147.471 77.049) (end 147.511 77.089) (width 0.254) (layer F.Cu) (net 7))
 (segment (start 146.0425 77.049) (end 146.5345 77.049) (width 0.254) (layer F.Cu) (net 7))
 (segment (start 146.7485 76.835) (end 147.6775 76.835) (width 0.254) (layer F.Cu) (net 7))
 (segment (start 146.5345 77.049) (end 146.7485 76.835) (width 0.254) (layer F.Cu) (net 7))
 (segment (start 147.6775 76.835) (end 147.6775 76.113) (width 0.254) (layer F.Cu) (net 7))
 (segment (start 146.685 75.311) (end 147.066 75.692) (width 0.254) (layer F.Cu) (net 7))
 (segment (start 147.2565 75.692) (end 147.6775 76.113) (width 0.254) (layer F.Cu) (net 7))
 (segment (start 147.066 75.692) (end 147.2565 75.692) (width 0.254) (layer F.Cu) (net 7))
 (segment (start 148.727905 75.311) (end 147.04421 75.311) (width 0.254) (layer B.Cu) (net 7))
 (segment (start 147.04421 75.311) (end 146.685 75.311) (width 0.254) (layer B.Cu) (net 7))
 (segment (start 149.181906 74.856999) (end 148.727905 75.311) (width 0.254) (layer B.Cu) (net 7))
 (segment (start 150.441001 75.159119) (end 150.138881 74.856999) (width 0.254) (layer B.Cu) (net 7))
 (segment (start 150.441001 80.444999) (end 150.441001 75.159119) (width 0.254) (layer B.Cu) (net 7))
 (segment (start 150.138881 74.856999) (end 149.181906 74.856999) (width 0.254) (layer B.Cu) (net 7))
 (segment (start 146.05 84.836) (end 150.441001 80.444999) (width 0.254) (layer B.Cu) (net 7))
 (segment (start 148.59 83.058) (end 148.59 84.836) (width 0.254) (layer F.Cu) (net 6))
 (segment (start 147.447 74.6125) (end 148.59 75.7555) (width 0.254) (layer F.Cu) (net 6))
 (segment (start 144.78 75.819) (end 145.9865 74.6125) (width 0.254) (layer F.Cu) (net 6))
 (segment (start 145.9865 74.6125) (end 147.447 74.6125) (width 0.254) (layer F.Cu) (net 6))
 (segment (start 144.78 76.5615) (end 144.78 75.819) (width 0.254) (layer F.Cu) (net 6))
 (segment (start 147.6775 78.867) (end 148.59 78.867) (width 0.254) (layer F.Cu) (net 6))
 (segment (start 148.59 78.867) (end 148.59 83.058) (width 0.254) (layer F.Cu) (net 6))
 (segment (start 148.59 75.7555) (end 148.59 78.867) (width 0.254) (layer F.Cu) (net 6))
 (via (at 142.748 82.042) (size 0.508) (drill 0.381) (layers F.Cu B.Cu) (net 2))
 (via (at 147.701 82.296) (size 0.508) (drill 0.381) (layers F.Cu B.Cu) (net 2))
 (segment (start 146.0425 80.424) (end 145.1865 81.28) (width 0.254) (layer F.Cu) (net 2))
 (segment (start 146.0425 80.049) (end 146.0425 80.424) (width 0.254) (layer F.Cu) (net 2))
 (segment (start 143.51 81.28) (end 142.748 82.042) (width 0.254) (layer F.Cu) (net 2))
 (segment (start 145.1865 81.28) (end 143.51 81.28) (width 0.254) (layer F.Cu) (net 2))
 (segment (start 143.51 81.28) (end 142.748 82.042) (width 0.254) (layer B.Cu) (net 2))
 (segment (start 144.055 81.28) (end 143.51 81.28) (width 0.254) (layer B.Cu) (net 2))
 (segment (start 147.6775 82.2725) (end 147.701 82.296) (width 0.254) (layer F.Cu) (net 2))
 (segment (start 147.6775 80.899) (end 147.6775 82.2725) (width 0.254) (layer F.Cu) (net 2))
 (segment (start 147.320001 82.676999) (end 147.701 82.296) (width 0.254) (layer B.Cu) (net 2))
 (segment (start 144.701999 82.676999) (end 147.320001 82.676999) (width 0.254) (layer B.Cu) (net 2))
 (segment (start 144.055 82.03) (end 144.701999 82.676999) (width 0.254) (layer B.Cu) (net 2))
 (segment (start 144.055 81.28) (end 144.055 82.03) (width 0.254) (layer B.Cu) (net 2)))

